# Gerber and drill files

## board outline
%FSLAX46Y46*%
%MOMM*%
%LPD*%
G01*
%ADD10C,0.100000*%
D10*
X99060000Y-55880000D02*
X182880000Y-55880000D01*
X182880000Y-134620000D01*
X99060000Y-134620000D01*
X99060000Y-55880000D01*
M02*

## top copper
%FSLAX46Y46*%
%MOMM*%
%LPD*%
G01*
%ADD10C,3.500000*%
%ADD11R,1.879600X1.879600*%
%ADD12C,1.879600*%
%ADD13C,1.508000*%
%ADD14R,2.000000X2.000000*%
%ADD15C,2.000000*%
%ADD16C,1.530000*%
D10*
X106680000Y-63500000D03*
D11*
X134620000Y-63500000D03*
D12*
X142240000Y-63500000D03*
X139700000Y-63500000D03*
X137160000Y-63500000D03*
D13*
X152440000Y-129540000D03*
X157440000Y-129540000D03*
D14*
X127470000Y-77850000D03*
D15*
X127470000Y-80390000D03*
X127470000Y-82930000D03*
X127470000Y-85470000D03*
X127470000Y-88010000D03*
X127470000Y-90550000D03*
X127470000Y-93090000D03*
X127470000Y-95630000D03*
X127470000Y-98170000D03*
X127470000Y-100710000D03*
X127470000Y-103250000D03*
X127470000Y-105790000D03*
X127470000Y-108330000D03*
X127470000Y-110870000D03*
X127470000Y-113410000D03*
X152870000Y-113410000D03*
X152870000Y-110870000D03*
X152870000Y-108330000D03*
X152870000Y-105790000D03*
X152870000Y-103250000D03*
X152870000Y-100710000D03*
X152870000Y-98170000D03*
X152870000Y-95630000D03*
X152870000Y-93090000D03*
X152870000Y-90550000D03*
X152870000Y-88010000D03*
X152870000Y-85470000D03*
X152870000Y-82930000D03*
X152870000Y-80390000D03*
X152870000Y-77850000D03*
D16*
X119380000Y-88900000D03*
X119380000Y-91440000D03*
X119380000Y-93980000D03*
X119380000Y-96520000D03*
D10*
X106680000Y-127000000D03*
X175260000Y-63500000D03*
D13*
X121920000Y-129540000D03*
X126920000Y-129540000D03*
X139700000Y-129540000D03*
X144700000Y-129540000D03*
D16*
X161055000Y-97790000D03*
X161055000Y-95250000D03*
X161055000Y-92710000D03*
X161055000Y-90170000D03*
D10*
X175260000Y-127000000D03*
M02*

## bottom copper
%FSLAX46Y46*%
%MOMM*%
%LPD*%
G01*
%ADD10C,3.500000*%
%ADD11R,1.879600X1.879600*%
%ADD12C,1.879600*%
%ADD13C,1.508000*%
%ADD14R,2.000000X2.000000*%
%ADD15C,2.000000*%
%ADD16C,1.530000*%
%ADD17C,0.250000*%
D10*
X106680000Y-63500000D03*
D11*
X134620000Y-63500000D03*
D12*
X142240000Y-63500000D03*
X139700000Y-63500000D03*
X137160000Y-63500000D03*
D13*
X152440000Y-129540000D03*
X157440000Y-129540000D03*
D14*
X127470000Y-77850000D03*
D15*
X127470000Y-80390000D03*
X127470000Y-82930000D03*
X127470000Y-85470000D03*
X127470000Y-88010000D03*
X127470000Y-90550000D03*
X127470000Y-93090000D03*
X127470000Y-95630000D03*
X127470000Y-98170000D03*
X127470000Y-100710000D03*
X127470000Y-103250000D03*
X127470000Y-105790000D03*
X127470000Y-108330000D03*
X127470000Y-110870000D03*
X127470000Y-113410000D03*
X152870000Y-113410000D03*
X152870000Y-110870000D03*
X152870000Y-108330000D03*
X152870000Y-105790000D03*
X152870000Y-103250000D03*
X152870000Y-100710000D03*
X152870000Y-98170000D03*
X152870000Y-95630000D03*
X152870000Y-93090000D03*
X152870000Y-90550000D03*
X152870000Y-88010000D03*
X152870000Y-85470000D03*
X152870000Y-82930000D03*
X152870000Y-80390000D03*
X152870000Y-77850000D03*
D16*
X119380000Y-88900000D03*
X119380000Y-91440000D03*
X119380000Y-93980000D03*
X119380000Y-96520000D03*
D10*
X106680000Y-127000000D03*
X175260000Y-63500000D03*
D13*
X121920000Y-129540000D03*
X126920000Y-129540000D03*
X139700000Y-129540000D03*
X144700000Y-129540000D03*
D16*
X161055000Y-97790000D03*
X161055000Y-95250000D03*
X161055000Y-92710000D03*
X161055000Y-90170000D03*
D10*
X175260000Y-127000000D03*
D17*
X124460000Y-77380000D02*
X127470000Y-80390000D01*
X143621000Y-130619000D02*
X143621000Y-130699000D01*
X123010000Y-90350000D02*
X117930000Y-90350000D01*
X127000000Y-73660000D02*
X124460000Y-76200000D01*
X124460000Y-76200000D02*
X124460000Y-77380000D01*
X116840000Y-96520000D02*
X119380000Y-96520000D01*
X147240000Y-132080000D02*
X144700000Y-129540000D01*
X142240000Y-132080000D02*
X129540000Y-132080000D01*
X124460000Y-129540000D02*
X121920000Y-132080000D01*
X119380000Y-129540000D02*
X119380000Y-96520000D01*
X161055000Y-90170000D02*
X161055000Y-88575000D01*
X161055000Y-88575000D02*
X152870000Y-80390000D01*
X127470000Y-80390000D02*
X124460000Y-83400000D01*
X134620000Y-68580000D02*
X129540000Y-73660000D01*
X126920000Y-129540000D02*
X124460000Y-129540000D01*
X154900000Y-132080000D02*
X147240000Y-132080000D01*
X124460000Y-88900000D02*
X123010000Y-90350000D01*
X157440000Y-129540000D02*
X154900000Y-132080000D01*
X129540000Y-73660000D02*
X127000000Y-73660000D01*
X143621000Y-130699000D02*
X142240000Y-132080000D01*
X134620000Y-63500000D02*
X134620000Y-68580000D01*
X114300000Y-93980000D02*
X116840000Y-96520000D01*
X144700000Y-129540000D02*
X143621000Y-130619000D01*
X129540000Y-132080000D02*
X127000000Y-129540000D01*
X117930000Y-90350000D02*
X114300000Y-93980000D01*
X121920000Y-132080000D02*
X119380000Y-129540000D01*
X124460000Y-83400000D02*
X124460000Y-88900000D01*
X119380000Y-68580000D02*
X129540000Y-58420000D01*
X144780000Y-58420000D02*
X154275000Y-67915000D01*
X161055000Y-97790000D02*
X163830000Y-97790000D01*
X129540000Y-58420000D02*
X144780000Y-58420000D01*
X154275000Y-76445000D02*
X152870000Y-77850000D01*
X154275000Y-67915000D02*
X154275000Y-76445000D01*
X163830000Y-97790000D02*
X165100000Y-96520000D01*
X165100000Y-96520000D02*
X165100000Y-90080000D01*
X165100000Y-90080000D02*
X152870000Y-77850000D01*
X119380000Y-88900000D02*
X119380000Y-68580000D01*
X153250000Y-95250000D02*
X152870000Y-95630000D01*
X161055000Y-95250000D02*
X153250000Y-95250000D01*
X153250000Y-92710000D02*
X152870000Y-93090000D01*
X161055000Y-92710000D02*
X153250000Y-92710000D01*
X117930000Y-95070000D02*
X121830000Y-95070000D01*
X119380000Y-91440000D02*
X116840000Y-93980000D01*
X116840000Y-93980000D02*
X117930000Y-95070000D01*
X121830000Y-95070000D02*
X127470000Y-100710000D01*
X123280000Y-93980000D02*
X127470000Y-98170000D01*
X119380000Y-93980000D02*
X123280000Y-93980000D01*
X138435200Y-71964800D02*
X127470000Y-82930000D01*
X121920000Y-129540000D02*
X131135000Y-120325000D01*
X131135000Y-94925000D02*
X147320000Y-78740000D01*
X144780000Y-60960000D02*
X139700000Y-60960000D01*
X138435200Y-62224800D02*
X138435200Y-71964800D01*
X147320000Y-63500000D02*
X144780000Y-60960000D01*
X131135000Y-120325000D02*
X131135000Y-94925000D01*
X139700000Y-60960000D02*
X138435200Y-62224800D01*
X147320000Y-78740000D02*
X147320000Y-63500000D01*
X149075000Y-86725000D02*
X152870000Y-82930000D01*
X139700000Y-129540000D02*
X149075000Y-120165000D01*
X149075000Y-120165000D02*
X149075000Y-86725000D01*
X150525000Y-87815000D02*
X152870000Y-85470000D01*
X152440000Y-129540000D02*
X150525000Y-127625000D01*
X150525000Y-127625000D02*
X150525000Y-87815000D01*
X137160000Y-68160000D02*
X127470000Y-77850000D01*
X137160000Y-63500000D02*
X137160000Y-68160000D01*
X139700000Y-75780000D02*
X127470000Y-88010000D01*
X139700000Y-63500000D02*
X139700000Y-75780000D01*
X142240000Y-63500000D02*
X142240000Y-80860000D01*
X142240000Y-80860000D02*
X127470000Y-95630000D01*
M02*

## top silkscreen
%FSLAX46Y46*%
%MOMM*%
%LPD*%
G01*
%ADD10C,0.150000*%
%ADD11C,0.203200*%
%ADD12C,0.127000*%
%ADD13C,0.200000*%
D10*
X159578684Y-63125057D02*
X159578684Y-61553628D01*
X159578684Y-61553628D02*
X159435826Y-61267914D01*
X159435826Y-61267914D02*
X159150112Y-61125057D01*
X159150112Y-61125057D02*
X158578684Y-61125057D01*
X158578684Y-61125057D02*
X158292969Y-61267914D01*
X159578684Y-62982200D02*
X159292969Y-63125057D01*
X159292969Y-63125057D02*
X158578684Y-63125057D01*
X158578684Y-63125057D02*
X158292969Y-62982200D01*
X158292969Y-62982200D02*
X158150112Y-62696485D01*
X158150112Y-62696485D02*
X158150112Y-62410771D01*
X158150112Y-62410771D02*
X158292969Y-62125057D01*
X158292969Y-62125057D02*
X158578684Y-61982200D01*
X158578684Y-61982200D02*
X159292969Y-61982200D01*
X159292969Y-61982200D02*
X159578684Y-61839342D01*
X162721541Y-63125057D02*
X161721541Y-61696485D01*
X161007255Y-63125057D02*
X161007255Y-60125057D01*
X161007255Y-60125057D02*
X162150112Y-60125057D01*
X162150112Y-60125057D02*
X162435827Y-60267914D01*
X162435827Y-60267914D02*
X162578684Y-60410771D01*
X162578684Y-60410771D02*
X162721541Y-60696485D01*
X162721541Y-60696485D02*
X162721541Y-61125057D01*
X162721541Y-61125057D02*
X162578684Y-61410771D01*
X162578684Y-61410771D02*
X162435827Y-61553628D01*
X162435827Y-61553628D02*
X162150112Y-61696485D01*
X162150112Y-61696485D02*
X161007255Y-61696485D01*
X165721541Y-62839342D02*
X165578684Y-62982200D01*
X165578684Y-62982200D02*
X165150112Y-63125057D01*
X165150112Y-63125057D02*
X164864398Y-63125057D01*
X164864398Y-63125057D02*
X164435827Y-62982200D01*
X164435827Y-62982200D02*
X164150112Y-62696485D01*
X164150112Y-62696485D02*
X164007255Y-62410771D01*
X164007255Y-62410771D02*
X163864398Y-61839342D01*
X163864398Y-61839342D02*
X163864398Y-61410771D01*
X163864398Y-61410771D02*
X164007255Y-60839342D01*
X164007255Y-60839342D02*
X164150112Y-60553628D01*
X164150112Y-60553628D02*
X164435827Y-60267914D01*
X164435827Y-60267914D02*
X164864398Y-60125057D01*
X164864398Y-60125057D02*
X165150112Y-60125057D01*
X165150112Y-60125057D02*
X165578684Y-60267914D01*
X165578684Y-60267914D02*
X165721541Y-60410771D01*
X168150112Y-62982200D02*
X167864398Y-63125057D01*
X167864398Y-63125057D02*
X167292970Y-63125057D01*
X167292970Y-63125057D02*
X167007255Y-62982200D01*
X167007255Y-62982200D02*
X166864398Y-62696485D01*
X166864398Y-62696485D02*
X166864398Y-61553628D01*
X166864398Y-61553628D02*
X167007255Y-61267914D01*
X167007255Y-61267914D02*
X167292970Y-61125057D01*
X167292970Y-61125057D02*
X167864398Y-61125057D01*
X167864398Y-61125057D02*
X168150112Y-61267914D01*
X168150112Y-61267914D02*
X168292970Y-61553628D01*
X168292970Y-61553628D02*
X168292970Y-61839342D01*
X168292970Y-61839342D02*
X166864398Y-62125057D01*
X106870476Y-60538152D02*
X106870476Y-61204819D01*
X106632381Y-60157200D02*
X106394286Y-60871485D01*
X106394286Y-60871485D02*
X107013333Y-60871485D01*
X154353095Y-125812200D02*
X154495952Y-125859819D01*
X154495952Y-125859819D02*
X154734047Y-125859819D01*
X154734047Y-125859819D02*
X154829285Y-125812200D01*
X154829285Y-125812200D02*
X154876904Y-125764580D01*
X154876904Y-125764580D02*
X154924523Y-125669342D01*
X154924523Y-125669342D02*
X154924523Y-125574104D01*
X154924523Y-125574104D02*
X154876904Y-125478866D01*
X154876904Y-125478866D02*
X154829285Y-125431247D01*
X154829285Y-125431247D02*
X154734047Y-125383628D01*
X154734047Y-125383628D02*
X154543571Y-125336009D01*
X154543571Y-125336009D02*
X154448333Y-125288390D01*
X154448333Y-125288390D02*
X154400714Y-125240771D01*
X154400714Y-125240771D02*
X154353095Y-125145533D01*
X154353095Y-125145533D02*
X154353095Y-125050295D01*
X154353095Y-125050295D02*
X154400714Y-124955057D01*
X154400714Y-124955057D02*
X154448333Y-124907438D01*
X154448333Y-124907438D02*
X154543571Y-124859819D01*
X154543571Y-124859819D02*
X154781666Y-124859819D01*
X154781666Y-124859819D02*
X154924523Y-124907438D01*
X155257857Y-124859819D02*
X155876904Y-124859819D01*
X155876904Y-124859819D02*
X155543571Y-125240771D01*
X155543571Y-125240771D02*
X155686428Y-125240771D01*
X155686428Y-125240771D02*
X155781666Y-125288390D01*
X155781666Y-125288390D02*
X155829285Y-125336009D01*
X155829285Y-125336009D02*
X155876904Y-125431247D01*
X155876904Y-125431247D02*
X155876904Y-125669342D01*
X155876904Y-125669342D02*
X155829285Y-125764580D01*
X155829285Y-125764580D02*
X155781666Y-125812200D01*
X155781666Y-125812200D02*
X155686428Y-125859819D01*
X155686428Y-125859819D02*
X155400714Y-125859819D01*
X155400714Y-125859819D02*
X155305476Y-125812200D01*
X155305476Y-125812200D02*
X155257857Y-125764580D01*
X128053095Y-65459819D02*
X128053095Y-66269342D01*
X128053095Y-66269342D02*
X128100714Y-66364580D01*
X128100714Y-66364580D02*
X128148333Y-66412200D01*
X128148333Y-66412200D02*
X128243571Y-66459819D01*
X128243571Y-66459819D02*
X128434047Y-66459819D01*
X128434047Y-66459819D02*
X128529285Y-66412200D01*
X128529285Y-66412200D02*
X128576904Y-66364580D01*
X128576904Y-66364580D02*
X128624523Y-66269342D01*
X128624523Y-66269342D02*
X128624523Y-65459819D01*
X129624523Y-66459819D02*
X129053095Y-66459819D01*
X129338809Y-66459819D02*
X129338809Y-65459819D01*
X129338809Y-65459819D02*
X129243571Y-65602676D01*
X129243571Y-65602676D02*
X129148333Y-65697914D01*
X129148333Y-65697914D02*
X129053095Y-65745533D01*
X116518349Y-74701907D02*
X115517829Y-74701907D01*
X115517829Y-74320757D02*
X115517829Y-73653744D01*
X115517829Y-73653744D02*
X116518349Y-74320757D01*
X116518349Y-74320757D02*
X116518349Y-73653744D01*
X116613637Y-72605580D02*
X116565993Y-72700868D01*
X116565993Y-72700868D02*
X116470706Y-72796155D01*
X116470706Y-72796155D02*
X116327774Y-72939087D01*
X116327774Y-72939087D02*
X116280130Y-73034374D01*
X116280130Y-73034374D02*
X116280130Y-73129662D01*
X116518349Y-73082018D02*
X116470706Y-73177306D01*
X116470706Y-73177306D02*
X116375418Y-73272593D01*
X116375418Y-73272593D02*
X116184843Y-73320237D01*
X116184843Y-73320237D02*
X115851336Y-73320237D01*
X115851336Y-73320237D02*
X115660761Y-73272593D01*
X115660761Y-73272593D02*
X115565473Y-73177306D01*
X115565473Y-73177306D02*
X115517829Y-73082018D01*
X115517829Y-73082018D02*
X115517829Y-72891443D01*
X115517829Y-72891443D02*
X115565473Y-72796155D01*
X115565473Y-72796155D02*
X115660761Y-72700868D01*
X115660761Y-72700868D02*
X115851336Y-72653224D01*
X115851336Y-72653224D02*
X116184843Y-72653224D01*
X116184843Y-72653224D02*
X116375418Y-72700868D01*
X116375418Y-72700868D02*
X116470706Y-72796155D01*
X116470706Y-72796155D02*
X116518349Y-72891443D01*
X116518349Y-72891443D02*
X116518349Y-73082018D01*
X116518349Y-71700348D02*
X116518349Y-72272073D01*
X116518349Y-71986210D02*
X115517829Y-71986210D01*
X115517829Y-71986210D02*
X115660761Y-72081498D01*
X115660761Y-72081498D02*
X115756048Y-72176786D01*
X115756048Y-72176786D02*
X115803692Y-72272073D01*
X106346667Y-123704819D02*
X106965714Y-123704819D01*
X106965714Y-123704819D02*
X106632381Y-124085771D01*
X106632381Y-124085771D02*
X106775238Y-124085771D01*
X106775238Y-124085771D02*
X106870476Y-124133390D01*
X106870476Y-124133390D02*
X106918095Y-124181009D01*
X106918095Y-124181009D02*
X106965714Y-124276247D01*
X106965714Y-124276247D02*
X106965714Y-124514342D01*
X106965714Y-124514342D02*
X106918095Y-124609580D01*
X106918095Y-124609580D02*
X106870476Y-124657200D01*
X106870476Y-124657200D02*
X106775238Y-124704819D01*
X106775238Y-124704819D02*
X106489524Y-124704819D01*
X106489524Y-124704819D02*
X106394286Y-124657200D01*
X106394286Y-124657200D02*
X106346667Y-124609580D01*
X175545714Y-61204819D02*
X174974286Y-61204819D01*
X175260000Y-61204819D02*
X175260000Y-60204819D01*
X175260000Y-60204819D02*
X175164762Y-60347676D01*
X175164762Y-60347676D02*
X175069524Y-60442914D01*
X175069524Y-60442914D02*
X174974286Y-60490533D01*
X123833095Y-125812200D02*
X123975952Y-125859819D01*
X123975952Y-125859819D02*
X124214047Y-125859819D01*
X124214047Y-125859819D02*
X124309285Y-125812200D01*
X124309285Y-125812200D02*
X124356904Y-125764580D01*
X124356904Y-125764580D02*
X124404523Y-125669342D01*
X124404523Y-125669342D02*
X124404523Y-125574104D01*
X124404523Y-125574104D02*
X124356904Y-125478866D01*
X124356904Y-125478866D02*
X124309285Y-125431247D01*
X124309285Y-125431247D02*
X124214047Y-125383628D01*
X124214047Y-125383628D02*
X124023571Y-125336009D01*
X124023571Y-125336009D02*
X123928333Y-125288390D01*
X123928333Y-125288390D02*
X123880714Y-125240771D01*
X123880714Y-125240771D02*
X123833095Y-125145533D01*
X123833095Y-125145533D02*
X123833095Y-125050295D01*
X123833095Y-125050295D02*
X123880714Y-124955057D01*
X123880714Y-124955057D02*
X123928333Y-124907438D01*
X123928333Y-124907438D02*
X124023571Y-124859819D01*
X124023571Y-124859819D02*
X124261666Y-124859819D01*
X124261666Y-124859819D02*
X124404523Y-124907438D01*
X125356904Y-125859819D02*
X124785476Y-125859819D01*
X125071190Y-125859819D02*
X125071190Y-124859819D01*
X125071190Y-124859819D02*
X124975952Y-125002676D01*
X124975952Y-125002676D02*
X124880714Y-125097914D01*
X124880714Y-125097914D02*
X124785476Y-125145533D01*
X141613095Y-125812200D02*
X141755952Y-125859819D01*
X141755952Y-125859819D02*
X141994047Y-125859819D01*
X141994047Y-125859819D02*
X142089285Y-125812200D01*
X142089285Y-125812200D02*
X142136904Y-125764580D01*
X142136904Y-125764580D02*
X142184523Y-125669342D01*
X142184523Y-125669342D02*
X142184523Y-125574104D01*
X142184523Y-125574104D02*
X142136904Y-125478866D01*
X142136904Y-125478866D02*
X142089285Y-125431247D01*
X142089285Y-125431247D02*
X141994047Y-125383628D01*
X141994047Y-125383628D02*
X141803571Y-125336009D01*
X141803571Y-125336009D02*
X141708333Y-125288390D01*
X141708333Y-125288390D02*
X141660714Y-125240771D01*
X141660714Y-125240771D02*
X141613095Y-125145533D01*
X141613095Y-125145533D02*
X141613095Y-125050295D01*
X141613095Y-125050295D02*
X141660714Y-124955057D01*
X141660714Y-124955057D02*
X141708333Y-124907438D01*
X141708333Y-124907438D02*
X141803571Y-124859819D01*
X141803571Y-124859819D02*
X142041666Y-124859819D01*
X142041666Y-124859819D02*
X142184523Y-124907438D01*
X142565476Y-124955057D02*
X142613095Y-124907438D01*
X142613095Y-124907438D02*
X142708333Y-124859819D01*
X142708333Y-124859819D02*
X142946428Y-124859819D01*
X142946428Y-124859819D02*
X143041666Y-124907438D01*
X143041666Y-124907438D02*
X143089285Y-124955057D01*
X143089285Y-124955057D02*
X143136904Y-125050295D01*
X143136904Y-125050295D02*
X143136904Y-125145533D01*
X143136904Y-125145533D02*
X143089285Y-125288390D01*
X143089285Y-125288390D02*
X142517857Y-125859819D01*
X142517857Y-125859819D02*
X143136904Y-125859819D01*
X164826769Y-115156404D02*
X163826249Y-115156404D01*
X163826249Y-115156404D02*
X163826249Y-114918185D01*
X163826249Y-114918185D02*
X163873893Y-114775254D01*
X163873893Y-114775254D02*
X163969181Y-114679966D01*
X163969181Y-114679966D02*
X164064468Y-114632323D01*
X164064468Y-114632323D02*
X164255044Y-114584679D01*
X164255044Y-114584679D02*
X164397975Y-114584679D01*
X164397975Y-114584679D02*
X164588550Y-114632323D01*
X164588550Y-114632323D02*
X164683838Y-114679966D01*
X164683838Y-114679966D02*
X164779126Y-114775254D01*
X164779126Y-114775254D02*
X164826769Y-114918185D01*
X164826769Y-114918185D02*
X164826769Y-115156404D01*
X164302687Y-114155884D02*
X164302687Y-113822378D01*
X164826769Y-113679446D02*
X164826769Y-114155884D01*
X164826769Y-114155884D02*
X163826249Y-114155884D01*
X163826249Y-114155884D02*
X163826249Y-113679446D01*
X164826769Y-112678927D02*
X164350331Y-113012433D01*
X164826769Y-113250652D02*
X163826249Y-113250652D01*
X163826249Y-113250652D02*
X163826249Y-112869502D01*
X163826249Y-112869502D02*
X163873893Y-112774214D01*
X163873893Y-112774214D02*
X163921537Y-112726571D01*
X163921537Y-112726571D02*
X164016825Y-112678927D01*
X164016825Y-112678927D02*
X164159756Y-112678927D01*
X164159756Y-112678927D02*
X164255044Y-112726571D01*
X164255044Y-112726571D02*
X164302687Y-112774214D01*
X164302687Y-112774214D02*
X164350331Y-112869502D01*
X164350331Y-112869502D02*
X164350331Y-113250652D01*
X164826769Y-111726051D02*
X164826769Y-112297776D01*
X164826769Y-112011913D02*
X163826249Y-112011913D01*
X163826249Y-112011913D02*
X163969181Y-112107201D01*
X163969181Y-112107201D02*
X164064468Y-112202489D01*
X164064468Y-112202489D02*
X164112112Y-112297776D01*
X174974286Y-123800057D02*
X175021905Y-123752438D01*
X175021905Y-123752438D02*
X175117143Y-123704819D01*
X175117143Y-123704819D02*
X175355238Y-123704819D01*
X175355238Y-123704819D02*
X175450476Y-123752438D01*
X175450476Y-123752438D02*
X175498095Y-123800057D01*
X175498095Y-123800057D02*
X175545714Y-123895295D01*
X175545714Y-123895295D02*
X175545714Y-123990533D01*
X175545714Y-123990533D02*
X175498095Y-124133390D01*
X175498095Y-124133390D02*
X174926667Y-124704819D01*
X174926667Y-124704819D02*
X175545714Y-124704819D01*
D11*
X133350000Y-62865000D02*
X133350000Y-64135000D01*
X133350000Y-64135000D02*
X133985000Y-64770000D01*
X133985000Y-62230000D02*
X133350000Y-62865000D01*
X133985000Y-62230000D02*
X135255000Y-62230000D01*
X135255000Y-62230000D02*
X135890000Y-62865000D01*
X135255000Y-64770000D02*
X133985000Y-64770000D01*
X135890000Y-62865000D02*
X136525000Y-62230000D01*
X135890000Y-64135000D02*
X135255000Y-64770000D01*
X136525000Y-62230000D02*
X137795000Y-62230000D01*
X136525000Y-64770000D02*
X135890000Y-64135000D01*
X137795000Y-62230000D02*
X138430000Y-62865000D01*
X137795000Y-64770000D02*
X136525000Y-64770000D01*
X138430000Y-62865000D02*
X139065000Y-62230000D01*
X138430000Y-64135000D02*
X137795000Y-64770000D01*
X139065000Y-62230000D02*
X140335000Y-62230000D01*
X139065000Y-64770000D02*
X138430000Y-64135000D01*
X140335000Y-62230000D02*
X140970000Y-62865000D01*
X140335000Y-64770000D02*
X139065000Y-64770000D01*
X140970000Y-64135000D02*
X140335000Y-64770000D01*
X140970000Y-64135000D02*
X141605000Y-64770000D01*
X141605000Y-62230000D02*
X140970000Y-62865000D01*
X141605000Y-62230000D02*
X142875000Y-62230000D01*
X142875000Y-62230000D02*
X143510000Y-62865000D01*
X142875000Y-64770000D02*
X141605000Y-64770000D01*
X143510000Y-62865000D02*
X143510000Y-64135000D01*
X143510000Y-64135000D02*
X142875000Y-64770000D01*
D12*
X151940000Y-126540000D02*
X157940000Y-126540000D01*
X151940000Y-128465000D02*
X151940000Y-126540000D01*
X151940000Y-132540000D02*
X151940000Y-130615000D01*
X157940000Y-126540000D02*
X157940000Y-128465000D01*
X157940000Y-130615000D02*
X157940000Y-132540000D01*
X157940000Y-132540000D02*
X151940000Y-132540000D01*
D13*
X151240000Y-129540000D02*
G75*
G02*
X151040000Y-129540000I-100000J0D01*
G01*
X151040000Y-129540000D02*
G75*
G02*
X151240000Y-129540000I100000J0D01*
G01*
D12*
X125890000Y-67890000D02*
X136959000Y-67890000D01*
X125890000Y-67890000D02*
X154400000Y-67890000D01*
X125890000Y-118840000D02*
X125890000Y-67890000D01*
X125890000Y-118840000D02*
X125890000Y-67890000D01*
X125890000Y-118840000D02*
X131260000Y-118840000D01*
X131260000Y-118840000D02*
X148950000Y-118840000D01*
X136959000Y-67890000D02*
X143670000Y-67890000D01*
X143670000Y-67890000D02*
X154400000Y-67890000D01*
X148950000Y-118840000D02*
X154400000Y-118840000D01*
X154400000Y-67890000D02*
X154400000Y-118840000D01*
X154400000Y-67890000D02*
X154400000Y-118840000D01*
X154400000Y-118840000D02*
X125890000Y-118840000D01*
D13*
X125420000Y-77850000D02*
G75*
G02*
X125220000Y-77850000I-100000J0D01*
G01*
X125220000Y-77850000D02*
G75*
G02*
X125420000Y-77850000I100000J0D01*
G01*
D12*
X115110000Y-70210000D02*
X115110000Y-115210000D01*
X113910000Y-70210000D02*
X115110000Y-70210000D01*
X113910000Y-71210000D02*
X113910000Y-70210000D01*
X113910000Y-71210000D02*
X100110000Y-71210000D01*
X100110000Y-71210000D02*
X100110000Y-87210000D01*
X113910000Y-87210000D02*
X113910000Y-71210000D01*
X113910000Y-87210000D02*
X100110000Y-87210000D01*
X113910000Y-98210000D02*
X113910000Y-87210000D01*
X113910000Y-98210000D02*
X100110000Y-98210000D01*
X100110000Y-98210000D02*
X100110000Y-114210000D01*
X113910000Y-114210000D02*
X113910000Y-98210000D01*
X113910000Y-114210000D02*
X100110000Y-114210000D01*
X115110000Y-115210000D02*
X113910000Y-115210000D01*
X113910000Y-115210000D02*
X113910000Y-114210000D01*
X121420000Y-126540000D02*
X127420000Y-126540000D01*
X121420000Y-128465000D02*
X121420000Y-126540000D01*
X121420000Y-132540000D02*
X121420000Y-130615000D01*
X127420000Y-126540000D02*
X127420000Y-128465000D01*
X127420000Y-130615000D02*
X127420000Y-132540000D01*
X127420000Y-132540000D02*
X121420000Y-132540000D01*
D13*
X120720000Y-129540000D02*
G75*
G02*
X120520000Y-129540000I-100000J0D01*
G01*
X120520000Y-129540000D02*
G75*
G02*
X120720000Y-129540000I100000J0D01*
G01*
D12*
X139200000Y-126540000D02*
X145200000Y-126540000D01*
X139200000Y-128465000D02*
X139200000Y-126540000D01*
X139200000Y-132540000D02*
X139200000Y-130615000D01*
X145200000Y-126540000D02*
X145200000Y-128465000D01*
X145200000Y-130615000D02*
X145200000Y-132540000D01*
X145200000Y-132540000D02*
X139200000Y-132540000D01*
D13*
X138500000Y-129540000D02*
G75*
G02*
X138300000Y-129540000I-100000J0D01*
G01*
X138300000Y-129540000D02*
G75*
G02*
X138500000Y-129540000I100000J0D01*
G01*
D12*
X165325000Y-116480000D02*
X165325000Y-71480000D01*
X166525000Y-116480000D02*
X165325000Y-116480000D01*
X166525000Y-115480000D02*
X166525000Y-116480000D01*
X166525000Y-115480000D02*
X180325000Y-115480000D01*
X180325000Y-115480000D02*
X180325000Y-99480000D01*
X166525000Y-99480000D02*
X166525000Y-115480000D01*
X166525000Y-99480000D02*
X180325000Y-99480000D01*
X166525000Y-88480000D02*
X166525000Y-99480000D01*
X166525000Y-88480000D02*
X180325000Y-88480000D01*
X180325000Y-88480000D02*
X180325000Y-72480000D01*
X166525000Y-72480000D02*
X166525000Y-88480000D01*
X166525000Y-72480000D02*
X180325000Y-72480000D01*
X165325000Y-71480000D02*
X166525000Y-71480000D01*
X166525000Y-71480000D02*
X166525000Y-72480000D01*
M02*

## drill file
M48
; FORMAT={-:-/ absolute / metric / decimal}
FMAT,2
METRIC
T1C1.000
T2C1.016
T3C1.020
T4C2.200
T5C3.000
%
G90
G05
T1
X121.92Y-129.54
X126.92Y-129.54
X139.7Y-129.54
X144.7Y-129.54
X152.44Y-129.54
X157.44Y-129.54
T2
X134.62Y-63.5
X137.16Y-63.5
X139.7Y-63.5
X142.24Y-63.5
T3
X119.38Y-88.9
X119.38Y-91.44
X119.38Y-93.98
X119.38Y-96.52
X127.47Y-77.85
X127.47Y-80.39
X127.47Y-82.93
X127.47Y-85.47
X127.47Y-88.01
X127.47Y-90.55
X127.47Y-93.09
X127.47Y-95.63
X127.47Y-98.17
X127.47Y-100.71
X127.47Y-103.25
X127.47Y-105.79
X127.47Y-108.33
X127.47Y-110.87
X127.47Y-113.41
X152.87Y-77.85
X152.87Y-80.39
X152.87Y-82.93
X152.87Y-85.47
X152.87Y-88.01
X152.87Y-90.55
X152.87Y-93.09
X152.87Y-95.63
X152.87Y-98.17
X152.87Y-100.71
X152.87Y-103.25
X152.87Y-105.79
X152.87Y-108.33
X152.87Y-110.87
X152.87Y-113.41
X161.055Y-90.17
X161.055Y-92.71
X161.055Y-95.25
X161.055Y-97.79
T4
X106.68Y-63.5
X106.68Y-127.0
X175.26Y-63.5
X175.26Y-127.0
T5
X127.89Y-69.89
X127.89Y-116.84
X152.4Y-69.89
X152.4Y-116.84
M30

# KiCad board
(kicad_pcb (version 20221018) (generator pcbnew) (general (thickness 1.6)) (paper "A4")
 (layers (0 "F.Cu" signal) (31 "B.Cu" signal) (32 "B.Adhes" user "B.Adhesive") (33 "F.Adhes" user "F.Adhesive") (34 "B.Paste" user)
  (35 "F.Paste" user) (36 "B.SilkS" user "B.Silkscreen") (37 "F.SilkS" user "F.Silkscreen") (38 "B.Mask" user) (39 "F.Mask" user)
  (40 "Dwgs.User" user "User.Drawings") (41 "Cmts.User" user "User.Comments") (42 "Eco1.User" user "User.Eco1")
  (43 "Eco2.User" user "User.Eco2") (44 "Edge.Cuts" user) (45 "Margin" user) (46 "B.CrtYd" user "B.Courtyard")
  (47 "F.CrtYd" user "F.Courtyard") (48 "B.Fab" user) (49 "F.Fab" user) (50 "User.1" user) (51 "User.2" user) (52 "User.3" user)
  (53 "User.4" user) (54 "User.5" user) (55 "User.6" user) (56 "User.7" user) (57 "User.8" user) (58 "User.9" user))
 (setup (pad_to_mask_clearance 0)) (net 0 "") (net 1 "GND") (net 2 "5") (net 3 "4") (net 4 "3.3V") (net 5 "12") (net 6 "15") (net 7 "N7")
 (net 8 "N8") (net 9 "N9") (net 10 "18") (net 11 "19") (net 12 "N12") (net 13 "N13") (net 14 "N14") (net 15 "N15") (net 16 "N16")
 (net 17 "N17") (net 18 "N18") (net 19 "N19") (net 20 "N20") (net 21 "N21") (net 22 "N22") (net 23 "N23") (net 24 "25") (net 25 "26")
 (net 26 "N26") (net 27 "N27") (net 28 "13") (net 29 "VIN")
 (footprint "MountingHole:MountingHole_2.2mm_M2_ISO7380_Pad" (layer "F.Cu") (at 106.68 63.5)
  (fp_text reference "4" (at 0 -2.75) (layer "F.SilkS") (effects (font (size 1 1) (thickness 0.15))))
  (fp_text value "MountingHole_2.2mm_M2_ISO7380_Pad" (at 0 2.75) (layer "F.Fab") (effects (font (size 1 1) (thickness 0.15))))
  (pad "1" thru_hole circle (at 0 0) (size 3.5 3.5) (drill 2.2) (layers "*.Cu" "*.Mask")))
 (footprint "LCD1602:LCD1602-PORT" (layer "F.Cu") (at 134.62 63.5)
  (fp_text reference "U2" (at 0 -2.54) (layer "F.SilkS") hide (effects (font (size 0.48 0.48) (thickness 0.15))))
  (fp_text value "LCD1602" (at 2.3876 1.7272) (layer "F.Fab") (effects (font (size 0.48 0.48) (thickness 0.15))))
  (fp_line (start -1.27 -0.635) (end -1.27 0.635) (stroke (width 0.2032) (type solid)) (layer "F.SilkS"))
  (fp_line (start -1.27 0.635) (end -0.635 1.27) (stroke (width 0.2032) (type solid)) (layer "F.SilkS"))
  (fp_line (start -0.635 -1.27) (end -1.27 -0.635) (stroke (width 0.2032) (type solid)) (layer "F.SilkS"))
  (fp_line (start -0.635 -1.27) (end 0.635 -1.27) (stroke (width 0.2032) (type solid)) (layer "F.SilkS"))
  (fp_line (start 0.635 -1.27) (end 1.27 -0.635) (stroke (width 0.2032) (type solid)) (layer "F.SilkS"))
  (fp_line (start 0.635 1.27) (end -0.635 1.27) (stroke (width 0.2032) (type solid)) (layer "F.SilkS"))
  (fp_line (start 1.27 -0.635) (end 1.905 -1.27) (stroke (width 0.2032) (type solid)) (layer "F.SilkS"))
  (fp_line (start 1.27 0.635) (end 0.635 1.27) (stroke (width 0.2032) (type solid)) (layer "F.SilkS"))
  (fp_line (start 1.905 -1.27) (end 3.175 -1.27) (stroke (width 0.2032) (type solid)) (layer "F.SilkS"))
  (fp_line (start 1.905 1.27) (end 1.27 0.635) (stroke (width 0.2032) (type solid)) (layer "F.SilkS"))
  (fp_line (start 3.175 -1.27) (end 3.81 -0.635) (stroke (width 0.2032) (type solid)) (layer "F.SilkS"))
  (fp_line (start 3.175 1.27) (end 1.905 1.27) (stroke (width 0.2032) (type solid)) (layer "F.SilkS"))
  (fp_line (start 3.81 -0.635) (end 4.445 -1.27) (stroke (width 0.2032) (type solid)) (layer "F.SilkS"))
  (fp_line (start 3.81 0.635) (end 3.175 1.27) (stroke (width 0.2032) (type solid)) (layer "F.SilkS"))
  (fp_line (start 4.445 -1.27) (end 5.715 -1.27) (stroke (width 0.2032) (type solid)) (layer "F.SilkS"))
  (fp_line (start 4.445 1.27) (end 3.81 0.635) (stroke (width 0.2032) (type solid)) (layer "F.SilkS"))
  (fp_line (start 5.715 -1.27) (end 6.35 -0.635) (stroke (width 0.2032) (type solid)) (layer "F.SilkS"))
  (fp_line (start 5.715 1.27) (end 4.445 1.27) (stroke (width 0.2032) (type solid)) (layer "F.SilkS"))
  (fp_line (start 6.35 0.635) (end 5.715 1.27) (stroke (width 0.2032) (type solid)) (layer "F.SilkS"))
  (fp_line (start 6.35 0.635) (end 6.985 1.27) (stroke (width 0.2032) (type solid)) (layer "F.SilkS"))
  (fp_line (start 6.985 -1.27) (end 6.35 -0.635) (stroke (width 0.2032) (type solid)) (layer "F.SilkS"))
  (fp_line (start 6.985 -1.27) (end 8.255 -1.27) (stroke (width 0.2032) (type solid)) (layer "F.SilkS"))
  (fp_line (start 8.255 -1.27) (end 8.89 -0.635) (stroke (width 0.2032) (type solid)) (layer "F.SilkS"))
  (fp_line (start 8.255 1.27) (end 6.985 1.27) (stroke (width 0.2032) (type solid)) (layer "F.SilkS"))
  (fp_line (start 8.89 -0.635) (end 8.89 0.635) (stroke (width 0.2032) (type solid)) (layer "F.SilkS"))
  (fp_line (start 8.89 0.635) (end 8.255 1.27) (stroke (width 0.2032) (type solid)) (layer "F.SilkS"))
  (pad "GND" thru_hole rect (at 0 0) (size 1.8796 1.8796) (drill 1.016) (layers "*.Cu" "*.Mask") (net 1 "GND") (solder_mask_margin 0.102))
  (pad "SCL" thru_hole circle (at 7.62 0) (size 1.8796 1.8796) (drill 1.016) (layers "*.Cu" "*.Mask") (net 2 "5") (solder_mask_margin 0.102))
  (pad "SDA" thru_hole circle (at 5.08 0) (size 1.8796 1.8796) (drill 1.016) (layers "*.Cu" "*.Mask") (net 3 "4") (solder_mask_margin 0.102))
  (pad "VCC" thru_hole circle (at 2.54 0) (size 1.8796 1.8796) (drill 1.016) (layers "*.Cu" "*.Mask") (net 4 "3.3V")
   (solder_mask_margin 0.102)))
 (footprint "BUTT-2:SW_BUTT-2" (layer "F.Cu") (at 154.94 129.54)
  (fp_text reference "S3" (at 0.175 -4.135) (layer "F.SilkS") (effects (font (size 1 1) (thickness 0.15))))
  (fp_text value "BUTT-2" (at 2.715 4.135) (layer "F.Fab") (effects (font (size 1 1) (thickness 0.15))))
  (fp_line (start -3 -3) (end 3 -3) (stroke (width 0.127) (type solid)) (layer "F.SilkS"))
  (fp_line (start -3 -1.075) (end -3 -3) (stroke (width 0.127) (type solid)) (layer "F.SilkS"))
  (fp_line (start -3 3) (end -3 1.075) (stroke (width 0.127) (type solid)) (layer "F.SilkS"))
  (fp_line (start 3 -3) (end 3 -1.075) (stroke (width 0.127) (type solid)) (layer "F.SilkS"))
  (fp_line (start 3 1.075) (end 3 3) (stroke (width 0.127) (type solid)) (layer "F.SilkS"))
  (fp_line (start 3 3) (end -3 3) (stroke (width 0.127) (type solid)) (layer "F.SilkS"))
  (fp_circle (center -3.8 0) (end -3.7 0) (stroke (width 0.2) (type solid)) (fill none) (layer "F.SilkS"))
  (pad "1" thru_hole circle (at -2.5 0) (size 1.508 1.508) (drill 1) (layers "*.Cu" "*.Mask") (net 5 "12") (solder_mask_margin 0.102))
  (pad "2" thru_hole circle (at 2.5 0) (size 1.508 1.508) (drill 1) (layers "*.Cu" "*.Mask") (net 1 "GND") (solder_mask_margin 0.102)))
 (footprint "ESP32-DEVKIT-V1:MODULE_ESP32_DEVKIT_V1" (layer "F.Cu") (at 140.17 93.365)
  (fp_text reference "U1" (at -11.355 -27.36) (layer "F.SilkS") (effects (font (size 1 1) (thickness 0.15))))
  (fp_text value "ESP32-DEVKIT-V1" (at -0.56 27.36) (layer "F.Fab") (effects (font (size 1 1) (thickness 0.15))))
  (fp_line (start -14.28 -25.475) (end -3.211 -25.475) (stroke (width 0.127) (type solid)) (layer "F.SilkS"))
  (fp_line (start -14.28 -25.475) (end 14.23 -25.475) (stroke (width 0.127) (type solid)) (layer "F.SilkS"))
  (fp_line (start -14.28 25.475) (end -14.28 -25.475) (stroke (width 0.127) (type solid)) (layer "F.SilkS"))
  (fp_line (start -14.28 25.475) (end -14.28 -25.475) (stroke (width 0.127) (type solid)) (layer "F.SilkS"))
  (fp_line (start -14.28 25.475) (end -8.91 25.475) (stroke (width 0.127) (type solid)) (layer "F.SilkS"))
  (fp_line (start -8.91 25.475) (end 8.78 25.475) (stroke (width 0.127) (type solid)) (layer "F.SilkS"))
  (fp_line (start -3.211 -25.475) (end 3.5 -25.475) (stroke (width 0.127) (type solid)) (layer "F.SilkS"))
  (fp_line (start 3.5 -25.475) (end 14.23 -25.475) (stroke (width 0.127) (type solid)) (layer "F.SilkS"))
  (fp_line (start 8.78 25.475) (end 14.23 25.475) (stroke (width 0.127) (type solid)) (layer "F.SilkS"))
  (fp_line (start 14.23 -25.475) (end 14.23 25.475) (stroke (width 0.127) (type solid)) (layer "F.SilkS"))
  (fp_line (start 14.23 -25.475) (end 14.23 25.475) (stroke (width 0.127) (type solid)) (layer "F.SilkS"))
  (fp_line (start 14.23 25.475) (end -14.28 25.475) (stroke (width 0.127) (type solid)) (layer "F.SilkS"))
  (fp_circle (center -14.85 -15.515) (end -14.75 -15.515) (stroke (width 0.2) (type solid)) (fill none) (layer "F.SilkS"))
  (pad "" np_thru_hole circle (at -12.28 -23.475) (size 3 3) (drill 3) (layers "*.Cu" "*.Mask"))
  (pad "" np_thru_hole circle (at -12.28 23.475) (size 3 3) (drill 3) (layers "*.Cu" "*.Mask"))
  (pad "" np_thru_hole circle (at 12.23 -23.475) (size 3 3) (drill 3) (layers "*.Cu" "*.Mask"))
  (pad "" np_thru_hole circle (at 12.23 23.475) (size 3 3) (drill 3) (layers "*.Cu" "*.Mask"))
  (pad "1" thru_hole rect (at -12.7 -15.515) (size 2 2) (drill 1.02) (layers "*.Cu" "*.Mask") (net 4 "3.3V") (solder_mask_margin 0.102))
  (pad "2" thru_hole circle (at -12.7 -12.975) (size 2 2) (drill 1.02) (layers "*.Cu" "*.Mask") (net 1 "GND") (solder_mask_margin 0.102))
  (pad "3" thru_hole circle (at -12.7 -10.435) (size 2 2) (drill 1.02) (layers "*.Cu" "*.Mask") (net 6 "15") (solder_mask_margin 0.102))
  (pad "4" thru_hole circle (at -12.7 -7.895) (size 2 2) (drill 1.02) (layers "*.Cu" "*.Mask") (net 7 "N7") (solder_mask_margin 0.102))
  (pad "5" thru_hole circle (at -12.7 -5.355) (size 2 2) (drill 1.02) (layers "*.Cu" "*.Mask") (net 3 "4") (solder_mask_margin 0.102))
  (pad "6" thru_hole circle (at -12.7 -2.815) (size 2 2) (drill 1.02) (layers "*.Cu" "*.Mask") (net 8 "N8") (solder_mask_margin 0.102))
  (pad "7" thru_hole circle (at -12.7 -0.275) (size 2 2) (drill 1.02) (layers "*.Cu" "*.Mask") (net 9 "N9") (solder_mask_margin 0.102))
  (pad "8" thru_hole circle (at -12.7 2.265) (size 2 2) (drill 1.02) (layers "*.Cu" "*.Mask") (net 2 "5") (solder_mask_margin 0.102))
  (pad "9" thru_hole circle (at -12.7 4.805) (size 2 2) (drill 1.02) (layers "*.Cu" "*.Mask") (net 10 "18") (solder_mask_margin 0.102))
  (pad "10" thru_hole circle (at -12.7 7.345) (size 2 2) (drill 1.02) (layers "*.Cu" "*.Mask") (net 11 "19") (solder_mask_margin 0.102))
  (pad "11" thru_hole circle (at -12.7 9.885) (size 2 2) (drill 1.02) (layers "*.Cu" "*.Mask") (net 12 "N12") (solder_mask_margin 0.102))
  (pad "12" thru_hole circle (at -12.7 12.425) (size 2 2) (drill 1.02) (layers "*.Cu" "*.Mask") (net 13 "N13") (solder_mask_margin 0.102))
  (pad "13" thru_hole circle (at -12.7 14.965) (size 2 2) (drill 1.02) (layers "*.Cu" "*.Mask") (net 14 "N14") (solder_mask_margin 0.102))
  (pad "14" thru_hole circle (at -12.7 17.505) (size 2 2) (drill 1.02) (layers "*.Cu" "*.Mask") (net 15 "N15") (solder_mask_margin 0.102))
  (pad "15" thru_hole circle (at -12.7 20.045) (size 2 2) (drill 1.02) (layers "*.Cu" "*.Mask") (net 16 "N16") (solder_mask_margin 0.102))
  (pad "16" thru_hole circle (at 12.7 20.045) (size 2 2) (drill 1.02) (layers "*.Cu" "*.Mask") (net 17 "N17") (solder_mask_margin 0.102))
  (pad "17" thru_hole circle (at 12.7 17.505) (size 2 2) (drill 1.02) (layers "*.Cu" "*.Mask") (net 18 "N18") (solder_mask_margin 0.102))
  (pad "18" thru_hole circle (at 12.7 14.965) (size 2 2) (drill 1.02) (layers "*.Cu" "*.Mask") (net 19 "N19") (solder_mask_margin 0.102))
  (pad "19" thru_hole circle (at 12.7 12.425) (size 2 2) (drill 1.02) (layers "*.Cu" "*.Mask") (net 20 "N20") (solder_mask_margin 0.102))
  (pad "20" thru_hole circle (at 12.7 9.885) (size 2 2) (drill 1.02) (layers "*.Cu" "*.Mask") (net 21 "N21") (solder_mask_margin 0.102))
  (pad "21" thru_hole circle (at 12.7 7.345) (size 2 2) (drill 1.02) (layers "*.Cu" "*.Mask") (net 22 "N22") (solder_mask_margin 0.102))
  (pad "22" thru_hole circle (at 12.7 4.805) (size 2 2) (drill 1.02) (layers "*.Cu" "*.Mask") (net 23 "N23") (solder_mask_margin 0.102))
  (pad "23" thru_hole circle (at 12.7 2.265) (size 2 2) (drill 1.02) (layers "*.Cu" "*.Mask") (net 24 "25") (solder_mask_margin 0.102))
  (pad "24" thru_hole circle (at 12.7 -0.275) (size 2 2) (drill 1.02) (layers "*.Cu" "*.Mask") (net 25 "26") (solder_mask_margin 0.102))
  (pad "25" thru_hole circle (at 12.7 -2.815) (size 2 2) (drill 1.02) (layers "*.Cu" "*.Mask") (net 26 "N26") (solder_mask_margin 0.102))
  (pad "26" thru_hole circle (at 12.7 -5.355) (size 2 2) (drill 1.02) (layers "*.Cu" "*.Mask") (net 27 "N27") (solder_mask_margin 0.102))
  (pad "27" thru_hole circle (at 12.7 -7.895) (size 2 2) (drill 1.02) (layers "*.Cu" "*.Mask") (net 5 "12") (solder_mask_margin 0.102))
  (pad "28" thru_hole circle (at 12.7 -10.435) (size 2 2) (drill 1.02) (layers "*.Cu" "*.Mask") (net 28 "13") (solder_mask_margin 0.102))
  (pad "29" thru_hole circle (at 12.7 -12.975) (size 2 2) (drill 1.02) (layers "*.Cu" "*.Mask") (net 1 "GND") (solder_mask_margin 0.102))
  (pad "30" thru_hole circle (at 12.7 -15.515) (size 2 2) (drill 1.02) (layers "*.Cu" "*.Mask") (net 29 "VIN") (solder_mask_margin 0.102))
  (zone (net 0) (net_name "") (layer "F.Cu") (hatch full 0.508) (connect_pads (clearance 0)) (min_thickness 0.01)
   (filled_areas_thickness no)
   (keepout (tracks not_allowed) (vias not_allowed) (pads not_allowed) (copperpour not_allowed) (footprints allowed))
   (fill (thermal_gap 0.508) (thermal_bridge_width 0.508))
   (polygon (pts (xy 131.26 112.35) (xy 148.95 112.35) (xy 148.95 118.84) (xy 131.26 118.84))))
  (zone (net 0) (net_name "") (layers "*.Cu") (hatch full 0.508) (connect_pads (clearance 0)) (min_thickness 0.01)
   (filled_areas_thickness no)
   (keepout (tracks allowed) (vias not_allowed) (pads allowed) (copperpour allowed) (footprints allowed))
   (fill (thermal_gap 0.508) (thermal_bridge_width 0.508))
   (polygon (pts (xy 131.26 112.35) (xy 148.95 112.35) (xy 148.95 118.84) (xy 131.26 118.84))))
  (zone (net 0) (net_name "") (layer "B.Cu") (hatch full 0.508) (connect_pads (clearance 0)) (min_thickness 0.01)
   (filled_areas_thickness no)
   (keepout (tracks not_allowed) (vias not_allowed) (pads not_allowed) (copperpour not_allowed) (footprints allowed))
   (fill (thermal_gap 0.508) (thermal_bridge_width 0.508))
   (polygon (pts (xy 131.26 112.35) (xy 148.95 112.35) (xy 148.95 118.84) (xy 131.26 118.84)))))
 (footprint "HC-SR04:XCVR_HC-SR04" (layer "F.Cu") (at 119.38 92.71 -90)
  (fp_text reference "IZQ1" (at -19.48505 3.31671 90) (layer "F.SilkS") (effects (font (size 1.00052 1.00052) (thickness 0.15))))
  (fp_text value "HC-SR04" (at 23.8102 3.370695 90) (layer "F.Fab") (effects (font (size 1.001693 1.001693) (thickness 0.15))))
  (fp_line (start -22.5 4.27) (end 22.5 4.27) (stroke (width 0.127) (type solid)) (layer "F.SilkS"))
  (fp_line (start -22.5 5.47) (end -22.5 4.27) (stroke (width 0.127) (type solid)) (layer "F.SilkS"))
  (fp_line (start -21.5 5.47) (end -22.5 5.47) (stroke (width 0.127) (type solid)) (layer "F.SilkS"))
  (fp_line (start -21.5 5.47) (end -21.5 19.27) (stroke (width 0.127) (type solid)) (layer "F.SilkS"))
  (fp_line (start -21.5 19.27) (end -5.5 19.27) (stroke (width 0.127) (type solid)) (layer "F.SilkS"))
  (fp_line (start -5.5 5.47) (end -21.5 5.47) (stroke (width 0.127) (type solid)) (layer "F.SilkS"))
  (fp_line (start -5.5 5.47) (end -5.5 19.27) (stroke (width 0.127) (type solid)) (layer "F.SilkS"))
  (fp_line (start 5.5 5.47) (end -5.5 5.47) (stroke (width 0.127) (type solid)) (layer "F.SilkS"))
  (fp_line (start 5.5 5.47) (end 5.5 19.27) (stroke (width 0.127) (type solid)) (layer "F.SilkS"))
  (fp_line (start 5.5 19.27) (end 21.5 19.27) (stroke (width 0.127) (type solid)) (layer "F.SilkS"))
  (fp_line (start 21.5 5.47) (end 5.5 5.47) (stroke (width 0.127) (type solid)) (layer "F.SilkS"))
  (fp_line (start 21.5 5.47) (end 21.5 19.27) (stroke (width 0.127) (type solid)) (layer "F.SilkS"))
  (fp_line (start 22.5 4.27) (end 22.5 5.47) (stroke (width 0.127) (type solid)) (layer "F.SilkS"))
  (fp_line (start 22.5 5.47) (end 21.5 5.47) (stroke (width 0.127) (type solid)) (layer "F.SilkS"))
  (pad "1" thru_hole circle (at -3.81 0 270) (size 1.53 1.53) (drill 1.02) (layers "*.Cu" "*.Mask") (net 29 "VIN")
   (solder_mask_margin 0.102))
  (pad "2" thru_hole circle (at -1.27 0 270) (size 1.53 1.53) (drill 1.02) (layers "*.Cu" "*.Mask") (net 11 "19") (solder_mask_margin 0.102))
  (pad "3" thru_hole circle (at 1.27 0 270) (size 1.53 1.53) (drill 1.02) (layers "*.Cu" "*.Mask") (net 10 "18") (solder_mask_margin 0.102))
  (pad "4" thru_hole circle (at 3.81 0 270) (size 1.53 1.53) (drill 1.02) (layers "*.Cu" "*.Mask") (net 1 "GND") (solder_mask_margin 0.102)))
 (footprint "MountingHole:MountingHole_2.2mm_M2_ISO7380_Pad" (layer "F.Cu") (at 106.68 127)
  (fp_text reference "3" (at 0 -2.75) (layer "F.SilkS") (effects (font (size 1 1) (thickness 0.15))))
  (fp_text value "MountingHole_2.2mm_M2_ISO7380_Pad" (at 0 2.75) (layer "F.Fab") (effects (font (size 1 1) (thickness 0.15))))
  (pad "1" thru_hole circle (at 0 0) (size 3.5 3.5) (drill 2.2) (layers "*.Cu" "*.Mask")))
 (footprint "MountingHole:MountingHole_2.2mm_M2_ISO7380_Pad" (layer "F.Cu") (at 175.26 63.5)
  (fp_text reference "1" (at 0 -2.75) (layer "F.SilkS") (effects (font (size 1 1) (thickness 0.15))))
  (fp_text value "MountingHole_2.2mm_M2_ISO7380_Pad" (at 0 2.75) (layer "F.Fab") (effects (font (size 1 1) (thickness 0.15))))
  (pad "1" thru_hole circle (at 0 0) (size 3.5 3.5) (drill 2.2) (layers "*.Cu" "*.Mask")))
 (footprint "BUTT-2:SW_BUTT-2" (layer "F.Cu") (at 124.42 129.54)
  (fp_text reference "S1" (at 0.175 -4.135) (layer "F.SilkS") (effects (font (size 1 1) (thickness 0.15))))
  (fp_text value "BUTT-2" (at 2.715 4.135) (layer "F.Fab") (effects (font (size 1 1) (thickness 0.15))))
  (fp_line (start -3 -3) (end 3 -3) (stroke (width 0.127) (type solid)) (layer "F.SilkS"))
  (fp_line (start -3 -1.075) (end -3 -3) (stroke (width 0.127) (type solid)) (layer "F.SilkS"))
  (fp_line (start -3 3) (end -3 1.075) (stroke (width 0.127) (type solid)) (layer "F.SilkS"))
  (fp_line (start 3 -3) (end 3 -1.075) (stroke (width 0.127) (type solid)) (layer "F.SilkS"))
  (fp_line (start 3 1.075) (end 3 3) (stroke (width 0.127) (type solid)) (layer "F.SilkS"))
  (fp_line (start 3 3) (end -3 3) (stroke (width 0.127) (type solid)) (layer "F.SilkS"))
  (fp_circle (center -3.8 0) (end -3.7 0) (stroke (width 0.2) (type solid)) (fill none) (layer "F.SilkS"))
  (pad "1" thru_hole circle (at -2.5 0) (size 1.508 1.508) (drill 1) (layers "*.Cu" "*.Mask") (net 6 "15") (solder_mask_margin 0.102))
  (pad "2" thru_hole circle (at 2.5 0) (size 1.508 1.508) (drill 1) (layers "*.Cu" "*.Mask") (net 1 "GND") (solder_mask_margin 0.102)))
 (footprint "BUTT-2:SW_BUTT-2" (layer "F.Cu") (at 142.2 129.54)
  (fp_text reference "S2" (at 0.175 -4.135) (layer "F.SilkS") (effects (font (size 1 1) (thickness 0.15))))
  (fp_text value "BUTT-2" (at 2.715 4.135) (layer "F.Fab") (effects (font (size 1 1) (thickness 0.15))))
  (fp_line (start -3 -3) (end 3 -3) (stroke (width 0.127) (type solid)) (layer "F.SilkS"))
  (fp_line (start -3 -1.075) (end -3 -3) (stroke (width 0.127) (type solid)) (layer "F.SilkS"))
  (fp_line (start -3 3) (end -3 1.075) (stroke (width 0.127) (type solid)) (layer "F.SilkS"))
  (fp_line (start 3 -3) (end 3 -1.075) (stroke (width 0.127) (type solid)) (layer "F.SilkS"))
  (fp_line (start 3 1.075) (end 3 3) (stroke (width 0.127) (type solid)) (layer "F.SilkS"))
  (fp_line (start 3 3) (end -3 3) (stroke (width 0.127) (type solid)) (layer "F.SilkS"))
  (fp_circle (center -3.8 0) (end -3.7 0) (stroke (width 0.2) (type solid)) (fill none) (layer "F.SilkS"))
  (pad "1" thru_hole circle (at -2.5 0) (size 1.508 1.508) (drill 1) (layers "*.Cu" "*.Mask") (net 28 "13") (solder_mask_margin 0.102))
  (pad "2" thru_hole circle (at 2.5 0) (size 1.508 1.508) (drill 1) (layers "*.Cu" "*.Mask") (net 1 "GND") (solder_mask_margin 0.102)))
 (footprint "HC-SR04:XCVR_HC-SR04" (layer "F.Cu") (at 161.055 93.98 90)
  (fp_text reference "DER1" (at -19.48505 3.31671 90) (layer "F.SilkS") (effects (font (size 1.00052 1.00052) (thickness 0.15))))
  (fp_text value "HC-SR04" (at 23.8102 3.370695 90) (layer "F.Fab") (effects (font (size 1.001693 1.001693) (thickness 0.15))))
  (fp_line (start -22.5 4.27) (end 22.5 4.27) (stroke (width 0.127) (type solid)) (layer "F.SilkS"))
  (fp_line (start -22.5 5.47) (end -22.5 4.27) (stroke (width 0.127) (type solid)) (layer "F.SilkS"))
  (fp_line (start -21.5 5.47) (end -22.5 5.47) (stroke (width 0.127) (type solid)) (layer "F.SilkS"))
  (fp_line (start -21.5 5.47) (end -21.5 19.27) (stroke (width 0.127) (type solid)) (layer "F.SilkS"))
  (fp_line (start -21.5 19.27) (end -5.5 19.27) (stroke (width 0.127) (type solid)) (layer "F.SilkS"))
  (fp_line (start -5.5 5.47) (end -21.5 5.47) (stroke (width 0.127) (type solid)) (layer "F.SilkS"))
  (fp_line (start -5.5 5.47) (end -5.5 19.27) (stroke (width 0.127) (type solid)) (layer "F.SilkS"))
  (fp_line (start 5.5 5.47) (end -5.5 5.47) (stroke (width 0.127) (type solid)) (layer "F.SilkS"))
  (fp_line (start 5.5 5.47) (end 5.5 19.27) (stroke (width 0.127) (type solid)) (layer "F.SilkS"))
  (fp_line (start 5.5 19.27) (end 21.5 19.27) (stroke (width 0.127) (type solid)) (layer "F.SilkS"))
  (fp_line (start 21.5 5.47) (end 5.5 5.47) (stroke (width 0.127) (type solid)) (layer "F.SilkS"))
  (fp_line (start 21.5 5.47) (end 21.5 19.27) (stroke (width 0.127) (type solid)) (layer "F.SilkS"))
  (fp_line (start 22.5 4.27) (end 22.5 5.47) (stroke (width 0.127) (type solid)) (layer "F.SilkS"))
  (fp_line (start 22.5 5.47) (end 21.5 5.47) (stroke (width 0.127) (type solid)) (layer "F.SilkS"))
  (pad "1" thru_hole circle (at -3.81 0 90) (size 1.53 1.53) (drill 1.02) (layers "*.Cu" "*.Mask") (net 29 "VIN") (solder_mask_margin 0.102))
  (pad "2" thru_hole circle (at -1.27 0 90) (size 1.53 1.53) (drill 1.02) (layers "*.Cu" "*.Mask") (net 24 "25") (solder_mask_margin 0.102))
  (pad "3" thru_hole circle (at 1.27 0 90) (size 1.53 1.53) (drill 1.02) (layers "*.Cu" "*.Mask") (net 25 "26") (solder_mask_margin 0.102))
  (pad "4" thru_hole circle (at 3.81 0 90) (size 1.53 1.53) (drill 1.02) (layers "*.Cu" "*.Mask") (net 1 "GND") (solder_mask_margin 0.102)))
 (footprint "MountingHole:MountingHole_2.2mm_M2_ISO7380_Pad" (layer "F.Cu") (at 175.26 127)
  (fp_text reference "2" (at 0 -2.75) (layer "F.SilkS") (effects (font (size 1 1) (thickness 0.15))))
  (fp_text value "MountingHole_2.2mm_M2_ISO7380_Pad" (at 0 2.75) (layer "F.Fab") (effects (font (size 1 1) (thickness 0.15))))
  (pad "1" thru_hole circle (at 0 0) (size 3.5 3.5) (drill 2.2) (layers "*.Cu" "*.Mask")))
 (gr_rect (start 99.06 55.88) (end 182.88 134.62) (stroke (width 0.1) (type default)) (fill none) (layer "Edge.Cuts"))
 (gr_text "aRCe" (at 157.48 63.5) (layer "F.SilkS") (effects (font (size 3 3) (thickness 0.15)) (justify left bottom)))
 (segment (start 124.46 77.38) (end 127.47 80.39) (width 0.25) (layer "B.Cu") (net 1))
 (segment (start 143.621 130.619) (end 143.621 130.699) (width 0.25) (layer "B.Cu") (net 1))
 (segment (start 123.01 90.35) (end 117.93 90.35) (width 0.25) (layer "B.Cu") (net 1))
 (segment (start 127 73.66) (end 124.46 76.2) (width 0.25) (layer "B.Cu") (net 1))
 (segment (start 124.46 76.2) (end 124.46 77.38) (width 0.25) (layer "B.Cu") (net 1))
 (segment (start 116.84 96.52) (end 119.38 96.52) (width 0.25) (layer "B.Cu") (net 1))
 (segment (start 147.24 132.08) (end 144.7 129.54) (width 0.25) (layer "B.Cu") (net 1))
 (segment (start 142.24 132.08) (end 129.54 132.08) (width 0.25) (layer "B.Cu") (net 1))
 (segment (start 124.46 129.54) (end 121.92 132.08) (width 0.25) (layer "B.Cu") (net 1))
 (segment (start 119.38 129.54) (end 119.38 96.52) (width 0.25) (layer "B.Cu") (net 1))
 (segment (start 161.055 90.17) (end 161.055 88.575) (width 0.25) (layer "B.Cu") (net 1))
 (segment (start 161.055 88.575) (end 152.87 80.39) (width 0.25) (layer "B.Cu") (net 1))
 (segment (start 127.47 80.39) (end 124.46 83.4) (width 0.25) (layer "B.Cu") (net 1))
 (segment (start 134.62 68.58) (end 129.54 73.66) (width 0.25) (layer "B.Cu") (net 1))
 (segment (start 126.92 129.54) (end 124.46 129.54) (width 0.25) (layer "B.Cu") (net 1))
 (segment (start 154.9 132.08) (end 147.24 132.08) (width 0.25) (layer "B.Cu") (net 1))
 (segment (start 124.46 88.9) (end 123.01 90.35) (width 0.25) (layer "B.Cu") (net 1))
 (segment (start 157.44 129.54) (end 154.9 132.08) (width 0.25) (layer "B.Cu") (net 1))
 (segment (start 129.54 73.66) (end 127 73.66) (width 0.25) (layer "B.Cu") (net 1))
 (segment (start 143.621 130.699) (end 142.24 132.08) (width 0.25) (layer "B.Cu") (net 1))
 (segment (start 134.62 63.5) (end 134.62 68.58) (width 0.25) (layer "B.Cu") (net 1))
 (segment (start 114.3 93.98) (end 116.84 96.52) (width 0.25) (layer "B.Cu") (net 1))
 (segment (start 144.7 129.54) (end 143.621 130.619) (width 0.25) (layer "B.Cu") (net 1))
 (segment (start 129.54 132.08) (end 127 129.54) (width 0.25) (layer "B.Cu") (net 1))
 (segment (start 117.93 90.35) (end 114.3 93.98) (width 0.25) (layer "B.Cu") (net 1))
 (segment (start 121.92 132.08) (end 119.38 129.54) (width 0.25) (layer "B.Cu") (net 1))
 (segment (start 124.46 83.4) (end 124.46 88.9) (width 0.25) (layer "B.Cu") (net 1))
 (segment (start 119.38 68.58) (end 129.54 58.42) (width 0.25) (layer "B.Cu") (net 29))
 (segment (start 144.78 58.42) (end 154.275 67.915) (width 0.25) (layer "B.Cu") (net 29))
 (segment (start 161.055 97.79) (end 163.83 97.79) (width 0.25) (layer "B.Cu") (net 29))
 (segment (start 129.54 58.42) (end 144.78 58.42) (width 0.25) (layer "B.Cu") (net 29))
 (segment (start 154.275 76.445) (end 152.87 77.85) (width 0.25) (layer "B.Cu") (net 29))
 (segment (start 154.275 67.915) (end 154.275 76.445) (width 0.25) (layer "B.Cu") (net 29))
 (segment (start 163.83 97.79) (end 165.1 96.52) (width 0.25) (layer "B.Cu") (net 29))
 (segment (start 165.1 96.52) (end 165.1 90.08) (width 0.25) (layer "B.Cu") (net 29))
 (segment (start 165.1 90.08) (end 152.87 77.85) (width 0.25) (layer "B.Cu") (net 29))
 (segment (start 119.38 88.9) (end 119.38 68.58) (width 0.25) (layer "B.Cu") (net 29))
 (segment (start 153.25 95.25) (end 152.87 95.63) (width 0.25) (layer "B.Cu") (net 24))
 (segment (start 161.055 95.25) (end 153.25 95.25) (width 0.25) (layer "B.Cu") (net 24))
 (segment (start 153.25 92.71) (end 152.87 93.09) (width 0.25) (layer "B.Cu") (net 25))
 (segment (start 161.055 92.71) (end 153.25 92.71) (width 0.25) (layer "B.Cu") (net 25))
 (segment (start 117.93 95.07) (end 121.83 95.07) (width 0.25) (layer "B.Cu") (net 11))
 (segment (start 119.38 91.44) (end 116.84 93.98) (width 0.25) (layer "B.Cu") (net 11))
 (segment (start 116.84 93.98) (end 117.93 95.07) (width 0.25) (layer "B.Cu") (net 11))
 (segment (start 121.83 95.07) (end 127.47 100.71) (width 0.25) (layer "B.Cu") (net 11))
 (segment (start 123.28 93.98) (end 127.47 98.17) (width 0.25) (layer "B.Cu") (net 10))
 (segment (start 119.38 93.98) (end 123.28 93.98) (width 0.25) (layer "B.Cu") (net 10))
 (segment (start 138.4352 71.9648) (end 127.47 82.93) (width 0.25) (layer "B.Cu") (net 6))
 (segment (start 121.92 129.54) (end 131.135 120.325) (width 0.25) (layer "B.Cu") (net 6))
 (segment (start 131.135 94.925) (end 147.32 78.74) (width 0.25) (layer "B.Cu") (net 6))
 (segment (start 144.78 60.96) (end 139.7 60.96) (width 0.25) (layer "B.Cu") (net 6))
 (segment (start 138.4352 62.2248) (end 138.4352 71.9648) (width 0.25) (layer "B.Cu") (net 6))
 (segment (start 147.32 63.5) (end 144.78 60.96) (width 0.25) (layer "B.Cu") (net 6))
 (segment (start 131.135 120.325) (end 131.135 94.925) (width 0.25) (layer "B.Cu") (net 6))
 (segment (start 139.7 60.96) (end 138.4352 62.2248) (width 0.25) (layer "B.Cu") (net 6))
 (segment (start 147.32 78.74) (end 147.32 63.5) (width 0.25) (layer "B.Cu") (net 6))
 (segment (start 149.075 86.725) (end 152.87 82.93) (width 0.25) (layer "B.Cu") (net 28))
 (segment (start 139.7 129.54) (end 149.075 120.165) (width 0.25) (layer "B.Cu") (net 28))
 (segment (start 149.075 120.165) (end 149.075 86.725) (width 0.25) (layer "B.Cu") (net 28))
 (segment (start 150.525 87.815) (end 152.87 85.47) (width 0.25) (layer "B.Cu") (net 5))
 (segment (start 152.44 129.54) (end 150.525 127.625) (width 0.25) (layer "B.Cu") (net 5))
 (segment (start 150.525 127.625) (end 150.525 87.815) (width 0.25) (layer "B.Cu") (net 5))
 (segment (start 137.16 68.16) (end 127.47 77.85) (width 0.25) (layer "B.Cu") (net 4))
 (segment (start 137.16 63.5) (end 137.16 68.16) (width 0.25) (layer "B.Cu") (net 4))
 (segment (start 139.7 75.78) (end 127.47 88.01) (width 0.25) (layer "B.Cu") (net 3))
 (segment (start 139.7 63.5) (end 139.7 75.78) (width 0.25) (layer "B.Cu") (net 3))
 (segment (start 142.24 63.5) (end 142.24 80.86) (width 0.25) (layer "B.Cu") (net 2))
 (segment (start 142.24 80.86) (end 127.47 95.63) (width 0.25) (layer "B.Cu") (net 2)))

